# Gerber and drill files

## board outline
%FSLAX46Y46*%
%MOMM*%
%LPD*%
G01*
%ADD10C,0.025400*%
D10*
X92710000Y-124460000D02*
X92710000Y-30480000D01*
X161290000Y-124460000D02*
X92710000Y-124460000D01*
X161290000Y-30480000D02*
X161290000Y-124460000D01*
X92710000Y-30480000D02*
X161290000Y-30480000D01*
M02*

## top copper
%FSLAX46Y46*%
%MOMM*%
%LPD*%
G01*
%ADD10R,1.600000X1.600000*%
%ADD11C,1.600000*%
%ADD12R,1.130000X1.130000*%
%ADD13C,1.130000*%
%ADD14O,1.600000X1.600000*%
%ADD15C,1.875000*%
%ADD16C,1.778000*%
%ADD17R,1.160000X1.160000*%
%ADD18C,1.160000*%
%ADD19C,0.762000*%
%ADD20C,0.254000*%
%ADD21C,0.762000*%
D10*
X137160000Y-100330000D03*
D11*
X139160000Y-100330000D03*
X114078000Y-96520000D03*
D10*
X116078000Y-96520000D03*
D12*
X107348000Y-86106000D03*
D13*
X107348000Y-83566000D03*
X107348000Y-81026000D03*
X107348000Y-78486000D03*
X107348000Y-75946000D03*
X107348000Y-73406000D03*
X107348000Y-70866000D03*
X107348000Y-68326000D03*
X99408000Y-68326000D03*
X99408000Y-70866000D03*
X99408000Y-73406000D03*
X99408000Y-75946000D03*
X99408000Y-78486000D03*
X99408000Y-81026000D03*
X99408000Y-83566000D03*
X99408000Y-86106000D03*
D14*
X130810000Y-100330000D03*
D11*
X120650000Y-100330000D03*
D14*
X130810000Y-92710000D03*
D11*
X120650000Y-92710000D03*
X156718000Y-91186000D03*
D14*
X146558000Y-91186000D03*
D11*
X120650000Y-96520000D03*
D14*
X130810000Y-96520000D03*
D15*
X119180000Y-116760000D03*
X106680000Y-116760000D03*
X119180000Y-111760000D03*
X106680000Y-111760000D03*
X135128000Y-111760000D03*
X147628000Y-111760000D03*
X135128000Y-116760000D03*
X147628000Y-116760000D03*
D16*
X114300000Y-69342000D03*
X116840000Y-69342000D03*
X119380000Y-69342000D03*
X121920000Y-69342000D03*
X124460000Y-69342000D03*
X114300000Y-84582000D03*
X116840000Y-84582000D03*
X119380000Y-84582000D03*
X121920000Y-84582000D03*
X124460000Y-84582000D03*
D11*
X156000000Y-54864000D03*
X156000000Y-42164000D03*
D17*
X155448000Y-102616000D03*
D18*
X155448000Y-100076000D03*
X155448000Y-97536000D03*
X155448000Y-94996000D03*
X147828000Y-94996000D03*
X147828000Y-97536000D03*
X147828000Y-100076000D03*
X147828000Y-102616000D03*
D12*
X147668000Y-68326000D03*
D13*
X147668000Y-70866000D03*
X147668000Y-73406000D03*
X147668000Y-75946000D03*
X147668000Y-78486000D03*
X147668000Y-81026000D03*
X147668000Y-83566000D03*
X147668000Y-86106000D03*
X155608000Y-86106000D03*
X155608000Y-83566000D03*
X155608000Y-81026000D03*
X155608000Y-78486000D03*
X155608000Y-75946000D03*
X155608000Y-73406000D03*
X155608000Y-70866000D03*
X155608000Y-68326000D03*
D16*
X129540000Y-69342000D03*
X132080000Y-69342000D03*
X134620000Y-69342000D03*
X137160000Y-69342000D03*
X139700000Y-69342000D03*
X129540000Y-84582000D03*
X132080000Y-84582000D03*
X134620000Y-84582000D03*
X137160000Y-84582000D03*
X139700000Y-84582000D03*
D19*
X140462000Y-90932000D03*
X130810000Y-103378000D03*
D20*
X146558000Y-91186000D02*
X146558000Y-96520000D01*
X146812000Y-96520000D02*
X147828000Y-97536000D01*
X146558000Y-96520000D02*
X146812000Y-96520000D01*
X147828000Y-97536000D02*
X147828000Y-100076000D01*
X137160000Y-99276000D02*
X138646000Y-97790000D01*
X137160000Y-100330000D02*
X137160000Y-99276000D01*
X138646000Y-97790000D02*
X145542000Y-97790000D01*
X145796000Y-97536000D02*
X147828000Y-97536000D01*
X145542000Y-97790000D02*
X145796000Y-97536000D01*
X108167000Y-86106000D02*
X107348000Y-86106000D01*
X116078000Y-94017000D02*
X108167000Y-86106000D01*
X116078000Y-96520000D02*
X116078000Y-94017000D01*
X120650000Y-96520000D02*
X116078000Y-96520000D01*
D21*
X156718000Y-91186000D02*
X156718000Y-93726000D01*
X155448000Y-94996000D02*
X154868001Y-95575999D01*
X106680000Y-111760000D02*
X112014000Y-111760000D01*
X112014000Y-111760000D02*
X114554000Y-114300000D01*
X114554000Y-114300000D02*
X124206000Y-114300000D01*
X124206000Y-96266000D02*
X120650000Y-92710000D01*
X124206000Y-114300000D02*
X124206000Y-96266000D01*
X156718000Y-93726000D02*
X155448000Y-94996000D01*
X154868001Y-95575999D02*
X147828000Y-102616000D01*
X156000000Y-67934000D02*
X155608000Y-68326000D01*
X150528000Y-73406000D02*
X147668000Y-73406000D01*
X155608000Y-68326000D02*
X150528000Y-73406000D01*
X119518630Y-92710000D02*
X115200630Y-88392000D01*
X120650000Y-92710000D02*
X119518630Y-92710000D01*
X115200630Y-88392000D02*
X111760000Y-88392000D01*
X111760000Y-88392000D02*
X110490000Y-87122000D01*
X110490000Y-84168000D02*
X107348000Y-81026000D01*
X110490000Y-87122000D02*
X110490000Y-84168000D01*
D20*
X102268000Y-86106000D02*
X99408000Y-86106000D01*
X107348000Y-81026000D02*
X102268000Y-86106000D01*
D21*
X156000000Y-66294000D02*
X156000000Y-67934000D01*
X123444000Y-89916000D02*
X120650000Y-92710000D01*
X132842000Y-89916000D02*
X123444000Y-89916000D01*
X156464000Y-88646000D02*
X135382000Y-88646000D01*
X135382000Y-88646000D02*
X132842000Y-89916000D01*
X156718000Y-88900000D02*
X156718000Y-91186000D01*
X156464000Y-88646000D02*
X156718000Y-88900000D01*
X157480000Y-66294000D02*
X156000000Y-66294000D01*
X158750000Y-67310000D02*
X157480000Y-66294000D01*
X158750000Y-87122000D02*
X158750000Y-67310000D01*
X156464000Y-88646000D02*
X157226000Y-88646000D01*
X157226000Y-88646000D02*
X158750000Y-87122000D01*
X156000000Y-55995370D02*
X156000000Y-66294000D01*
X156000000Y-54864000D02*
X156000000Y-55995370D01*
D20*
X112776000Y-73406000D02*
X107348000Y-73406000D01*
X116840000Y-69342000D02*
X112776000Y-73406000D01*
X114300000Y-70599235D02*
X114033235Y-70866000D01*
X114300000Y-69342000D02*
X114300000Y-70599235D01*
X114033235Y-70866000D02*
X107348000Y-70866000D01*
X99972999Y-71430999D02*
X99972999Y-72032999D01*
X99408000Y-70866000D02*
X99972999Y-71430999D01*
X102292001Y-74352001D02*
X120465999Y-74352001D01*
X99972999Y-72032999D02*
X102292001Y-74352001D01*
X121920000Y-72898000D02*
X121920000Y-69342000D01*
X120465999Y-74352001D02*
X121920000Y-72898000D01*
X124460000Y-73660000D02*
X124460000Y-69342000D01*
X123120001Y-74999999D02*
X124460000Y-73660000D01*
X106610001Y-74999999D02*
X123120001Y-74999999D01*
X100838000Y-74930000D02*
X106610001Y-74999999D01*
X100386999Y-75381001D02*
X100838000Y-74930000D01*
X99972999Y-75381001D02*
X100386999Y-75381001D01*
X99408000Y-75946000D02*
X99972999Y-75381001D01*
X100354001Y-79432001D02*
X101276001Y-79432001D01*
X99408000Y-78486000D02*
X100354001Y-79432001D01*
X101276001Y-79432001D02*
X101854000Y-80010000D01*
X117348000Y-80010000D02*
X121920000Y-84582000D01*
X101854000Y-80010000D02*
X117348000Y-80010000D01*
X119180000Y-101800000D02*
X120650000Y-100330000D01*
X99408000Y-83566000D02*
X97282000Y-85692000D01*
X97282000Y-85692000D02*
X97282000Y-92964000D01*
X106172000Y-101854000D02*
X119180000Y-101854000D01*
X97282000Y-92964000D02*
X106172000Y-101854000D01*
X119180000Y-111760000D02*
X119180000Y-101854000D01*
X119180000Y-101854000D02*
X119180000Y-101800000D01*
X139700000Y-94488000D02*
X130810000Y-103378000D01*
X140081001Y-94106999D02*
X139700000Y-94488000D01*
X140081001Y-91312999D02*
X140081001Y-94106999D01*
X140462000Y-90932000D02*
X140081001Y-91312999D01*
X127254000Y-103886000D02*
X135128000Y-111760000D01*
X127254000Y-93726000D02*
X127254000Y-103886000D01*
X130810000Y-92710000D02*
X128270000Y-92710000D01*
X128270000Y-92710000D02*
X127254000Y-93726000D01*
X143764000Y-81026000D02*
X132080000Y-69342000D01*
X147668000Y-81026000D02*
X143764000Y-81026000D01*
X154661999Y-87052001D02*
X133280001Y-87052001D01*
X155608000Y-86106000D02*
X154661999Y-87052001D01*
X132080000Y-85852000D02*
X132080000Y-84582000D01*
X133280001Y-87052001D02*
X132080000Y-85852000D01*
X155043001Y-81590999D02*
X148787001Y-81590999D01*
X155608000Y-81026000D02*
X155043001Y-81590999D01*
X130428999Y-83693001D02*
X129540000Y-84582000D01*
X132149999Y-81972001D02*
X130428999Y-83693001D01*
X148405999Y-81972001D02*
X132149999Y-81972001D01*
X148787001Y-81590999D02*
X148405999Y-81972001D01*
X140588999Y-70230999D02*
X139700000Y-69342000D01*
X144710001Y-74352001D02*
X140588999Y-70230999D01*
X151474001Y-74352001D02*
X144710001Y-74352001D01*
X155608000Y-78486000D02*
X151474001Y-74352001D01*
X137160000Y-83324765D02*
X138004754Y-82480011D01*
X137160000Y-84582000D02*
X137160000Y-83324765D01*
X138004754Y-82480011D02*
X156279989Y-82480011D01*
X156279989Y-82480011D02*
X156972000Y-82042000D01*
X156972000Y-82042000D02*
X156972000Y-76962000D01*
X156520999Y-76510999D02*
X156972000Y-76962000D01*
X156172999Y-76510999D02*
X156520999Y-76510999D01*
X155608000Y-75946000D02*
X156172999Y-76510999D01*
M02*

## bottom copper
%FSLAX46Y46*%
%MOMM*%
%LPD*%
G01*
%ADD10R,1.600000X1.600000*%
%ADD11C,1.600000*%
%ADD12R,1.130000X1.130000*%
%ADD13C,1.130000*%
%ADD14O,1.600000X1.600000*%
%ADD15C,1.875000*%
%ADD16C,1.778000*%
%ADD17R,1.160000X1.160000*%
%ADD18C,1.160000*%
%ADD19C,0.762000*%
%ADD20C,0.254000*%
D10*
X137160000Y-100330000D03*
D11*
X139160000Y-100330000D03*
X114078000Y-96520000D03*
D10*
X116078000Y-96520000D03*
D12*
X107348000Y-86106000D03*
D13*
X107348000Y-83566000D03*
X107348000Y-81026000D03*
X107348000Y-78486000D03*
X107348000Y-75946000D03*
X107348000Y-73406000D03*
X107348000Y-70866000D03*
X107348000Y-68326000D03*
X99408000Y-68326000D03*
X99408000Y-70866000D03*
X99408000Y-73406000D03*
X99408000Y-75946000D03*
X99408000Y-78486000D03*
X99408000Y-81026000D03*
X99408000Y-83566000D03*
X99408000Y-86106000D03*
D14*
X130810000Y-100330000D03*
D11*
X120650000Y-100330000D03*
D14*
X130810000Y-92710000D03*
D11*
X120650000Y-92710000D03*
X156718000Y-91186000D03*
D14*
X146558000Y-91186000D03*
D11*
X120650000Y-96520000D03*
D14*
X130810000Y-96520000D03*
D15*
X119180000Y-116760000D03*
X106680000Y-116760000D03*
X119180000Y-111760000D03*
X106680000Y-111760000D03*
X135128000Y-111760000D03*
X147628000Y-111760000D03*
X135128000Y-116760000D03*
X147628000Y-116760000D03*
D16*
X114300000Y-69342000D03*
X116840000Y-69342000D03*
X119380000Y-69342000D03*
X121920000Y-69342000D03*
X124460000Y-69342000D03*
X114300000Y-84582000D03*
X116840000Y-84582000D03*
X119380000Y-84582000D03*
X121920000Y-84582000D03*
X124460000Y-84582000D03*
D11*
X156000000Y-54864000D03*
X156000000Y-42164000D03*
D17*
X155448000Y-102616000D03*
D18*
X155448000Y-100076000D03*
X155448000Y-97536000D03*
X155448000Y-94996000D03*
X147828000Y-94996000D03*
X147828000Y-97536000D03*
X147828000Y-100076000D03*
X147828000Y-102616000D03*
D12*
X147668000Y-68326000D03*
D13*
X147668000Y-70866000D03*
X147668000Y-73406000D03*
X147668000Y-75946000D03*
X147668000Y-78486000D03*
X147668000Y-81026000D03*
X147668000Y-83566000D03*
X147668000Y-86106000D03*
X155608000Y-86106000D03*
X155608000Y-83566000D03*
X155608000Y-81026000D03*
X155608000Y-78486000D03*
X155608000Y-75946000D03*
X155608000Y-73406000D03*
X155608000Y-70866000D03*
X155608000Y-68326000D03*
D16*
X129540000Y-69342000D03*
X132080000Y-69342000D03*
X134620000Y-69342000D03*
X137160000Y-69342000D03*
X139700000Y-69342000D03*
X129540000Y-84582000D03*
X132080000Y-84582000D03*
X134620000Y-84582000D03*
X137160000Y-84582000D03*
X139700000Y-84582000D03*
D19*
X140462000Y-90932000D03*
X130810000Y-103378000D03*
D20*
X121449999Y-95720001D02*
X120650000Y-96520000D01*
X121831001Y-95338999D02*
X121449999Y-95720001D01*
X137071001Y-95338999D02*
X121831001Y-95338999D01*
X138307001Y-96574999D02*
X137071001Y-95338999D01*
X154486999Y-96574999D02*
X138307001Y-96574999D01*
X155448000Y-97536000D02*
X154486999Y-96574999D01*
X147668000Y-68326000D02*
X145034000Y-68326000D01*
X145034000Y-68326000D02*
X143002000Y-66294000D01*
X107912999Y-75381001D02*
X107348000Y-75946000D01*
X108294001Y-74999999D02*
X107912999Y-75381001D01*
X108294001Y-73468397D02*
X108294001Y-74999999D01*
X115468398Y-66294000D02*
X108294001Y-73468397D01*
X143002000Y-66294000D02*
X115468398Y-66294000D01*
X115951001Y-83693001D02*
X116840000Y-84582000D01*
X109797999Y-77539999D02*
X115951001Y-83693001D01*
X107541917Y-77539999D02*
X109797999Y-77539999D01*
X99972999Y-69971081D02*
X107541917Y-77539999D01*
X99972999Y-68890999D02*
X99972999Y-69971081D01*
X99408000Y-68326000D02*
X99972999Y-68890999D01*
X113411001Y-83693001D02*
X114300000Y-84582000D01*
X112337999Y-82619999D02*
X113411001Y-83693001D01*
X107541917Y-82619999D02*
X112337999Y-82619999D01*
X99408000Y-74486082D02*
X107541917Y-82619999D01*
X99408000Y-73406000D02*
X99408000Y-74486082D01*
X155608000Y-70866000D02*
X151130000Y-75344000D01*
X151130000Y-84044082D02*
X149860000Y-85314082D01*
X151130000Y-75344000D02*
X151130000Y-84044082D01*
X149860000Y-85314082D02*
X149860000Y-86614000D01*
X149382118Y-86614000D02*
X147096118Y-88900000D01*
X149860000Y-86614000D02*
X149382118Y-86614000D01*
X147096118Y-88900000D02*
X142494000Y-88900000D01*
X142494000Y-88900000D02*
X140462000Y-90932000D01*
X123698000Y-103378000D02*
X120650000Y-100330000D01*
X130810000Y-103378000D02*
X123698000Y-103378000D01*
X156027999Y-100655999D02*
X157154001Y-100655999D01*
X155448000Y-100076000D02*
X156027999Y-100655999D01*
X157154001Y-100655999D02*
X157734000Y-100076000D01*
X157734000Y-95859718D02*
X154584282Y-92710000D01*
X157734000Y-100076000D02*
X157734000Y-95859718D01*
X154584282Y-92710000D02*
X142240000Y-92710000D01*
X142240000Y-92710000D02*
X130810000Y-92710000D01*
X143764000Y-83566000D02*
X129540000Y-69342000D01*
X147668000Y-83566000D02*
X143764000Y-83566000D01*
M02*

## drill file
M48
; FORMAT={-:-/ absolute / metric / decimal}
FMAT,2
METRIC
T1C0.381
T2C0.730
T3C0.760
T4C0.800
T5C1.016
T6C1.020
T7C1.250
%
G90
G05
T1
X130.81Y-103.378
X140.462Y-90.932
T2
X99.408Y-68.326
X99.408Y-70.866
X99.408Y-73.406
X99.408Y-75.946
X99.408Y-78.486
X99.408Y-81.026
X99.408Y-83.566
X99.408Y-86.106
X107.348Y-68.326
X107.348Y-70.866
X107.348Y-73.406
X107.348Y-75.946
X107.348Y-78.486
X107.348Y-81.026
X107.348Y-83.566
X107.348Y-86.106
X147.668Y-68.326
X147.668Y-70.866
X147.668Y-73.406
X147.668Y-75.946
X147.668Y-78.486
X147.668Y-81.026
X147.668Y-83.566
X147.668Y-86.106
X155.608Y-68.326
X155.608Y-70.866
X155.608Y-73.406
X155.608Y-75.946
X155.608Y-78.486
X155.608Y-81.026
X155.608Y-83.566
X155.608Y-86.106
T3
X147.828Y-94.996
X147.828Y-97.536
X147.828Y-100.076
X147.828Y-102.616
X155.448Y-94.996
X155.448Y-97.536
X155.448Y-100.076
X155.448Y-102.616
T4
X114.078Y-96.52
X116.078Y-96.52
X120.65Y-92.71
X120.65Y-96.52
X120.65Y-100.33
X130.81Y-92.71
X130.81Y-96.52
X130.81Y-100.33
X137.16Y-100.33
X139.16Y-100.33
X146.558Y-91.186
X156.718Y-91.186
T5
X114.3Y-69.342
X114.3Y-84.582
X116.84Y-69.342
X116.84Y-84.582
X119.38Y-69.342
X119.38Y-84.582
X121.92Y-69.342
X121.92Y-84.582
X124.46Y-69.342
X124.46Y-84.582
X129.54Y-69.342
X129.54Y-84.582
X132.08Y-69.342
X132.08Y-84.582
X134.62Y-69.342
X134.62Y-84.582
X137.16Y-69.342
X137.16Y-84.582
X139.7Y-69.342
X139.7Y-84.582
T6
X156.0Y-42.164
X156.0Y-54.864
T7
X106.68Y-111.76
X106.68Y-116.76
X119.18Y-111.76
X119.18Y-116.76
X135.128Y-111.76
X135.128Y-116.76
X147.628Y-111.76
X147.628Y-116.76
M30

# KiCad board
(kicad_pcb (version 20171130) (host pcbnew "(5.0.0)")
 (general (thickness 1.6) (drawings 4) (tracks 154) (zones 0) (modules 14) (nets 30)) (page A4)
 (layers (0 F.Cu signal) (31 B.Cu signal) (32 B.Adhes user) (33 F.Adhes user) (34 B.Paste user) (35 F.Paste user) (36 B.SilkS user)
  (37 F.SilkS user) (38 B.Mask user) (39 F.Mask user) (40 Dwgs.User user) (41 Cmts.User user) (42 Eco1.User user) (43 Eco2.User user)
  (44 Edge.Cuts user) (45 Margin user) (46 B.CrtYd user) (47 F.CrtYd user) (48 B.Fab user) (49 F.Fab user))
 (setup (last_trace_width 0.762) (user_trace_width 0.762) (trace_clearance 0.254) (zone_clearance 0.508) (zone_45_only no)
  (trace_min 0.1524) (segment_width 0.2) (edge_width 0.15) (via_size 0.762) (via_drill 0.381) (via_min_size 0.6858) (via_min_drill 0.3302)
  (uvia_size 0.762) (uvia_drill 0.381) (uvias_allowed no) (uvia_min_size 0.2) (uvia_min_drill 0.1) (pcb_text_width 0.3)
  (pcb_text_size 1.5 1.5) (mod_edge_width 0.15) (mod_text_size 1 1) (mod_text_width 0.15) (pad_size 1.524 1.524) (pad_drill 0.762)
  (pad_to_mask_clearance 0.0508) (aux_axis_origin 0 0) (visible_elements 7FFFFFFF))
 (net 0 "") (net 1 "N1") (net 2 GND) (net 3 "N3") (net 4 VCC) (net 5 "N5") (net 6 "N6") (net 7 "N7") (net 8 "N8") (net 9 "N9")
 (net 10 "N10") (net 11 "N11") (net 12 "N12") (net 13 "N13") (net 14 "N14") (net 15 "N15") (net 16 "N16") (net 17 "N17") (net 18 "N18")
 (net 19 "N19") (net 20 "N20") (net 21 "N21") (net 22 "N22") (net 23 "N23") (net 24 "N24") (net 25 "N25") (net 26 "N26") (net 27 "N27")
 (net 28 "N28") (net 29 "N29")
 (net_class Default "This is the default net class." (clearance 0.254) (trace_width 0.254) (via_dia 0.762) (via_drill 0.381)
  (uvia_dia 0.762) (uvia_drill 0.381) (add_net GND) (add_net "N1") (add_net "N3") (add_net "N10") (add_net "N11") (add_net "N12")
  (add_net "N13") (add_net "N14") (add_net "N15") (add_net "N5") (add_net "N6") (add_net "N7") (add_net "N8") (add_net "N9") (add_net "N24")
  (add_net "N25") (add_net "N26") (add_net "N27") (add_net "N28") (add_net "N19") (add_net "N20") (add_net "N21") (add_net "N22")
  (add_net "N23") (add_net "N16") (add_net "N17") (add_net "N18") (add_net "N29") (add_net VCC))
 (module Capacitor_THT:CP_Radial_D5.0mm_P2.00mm (layer F.Cu) (at 137.16 100.33)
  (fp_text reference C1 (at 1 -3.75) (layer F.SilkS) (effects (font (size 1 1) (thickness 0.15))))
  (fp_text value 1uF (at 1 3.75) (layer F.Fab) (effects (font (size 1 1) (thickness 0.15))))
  (pad 1 thru_hole rect (at 0 0) (size 1.6 1.6) (drill 0.8) (layers *.Cu *.Mask) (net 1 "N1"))
  (pad 2 thru_hole circle (at 2 0) (size 1.6 1.6) (drill 0.8) (layers *.Cu *.Mask) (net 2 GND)))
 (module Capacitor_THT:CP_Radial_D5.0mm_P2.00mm (layer F.Cu) (at 116.078 96.52 180)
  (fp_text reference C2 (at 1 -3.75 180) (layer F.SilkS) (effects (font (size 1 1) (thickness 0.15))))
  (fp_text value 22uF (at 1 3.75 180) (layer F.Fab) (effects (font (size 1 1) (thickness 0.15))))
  (pad 2 thru_hole circle (at 2 0 180) (size 1.6 1.6) (drill 0.8) (layers *.Cu *.Mask) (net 2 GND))
  (pad 1 thru_hole rect (at 0 0 180) (size 1.6 1.6) (drill 0.8) (layers *.Cu *.Mask) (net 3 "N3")))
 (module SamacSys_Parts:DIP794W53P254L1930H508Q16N (layer F.Cu) (at 103.378 77.216 180)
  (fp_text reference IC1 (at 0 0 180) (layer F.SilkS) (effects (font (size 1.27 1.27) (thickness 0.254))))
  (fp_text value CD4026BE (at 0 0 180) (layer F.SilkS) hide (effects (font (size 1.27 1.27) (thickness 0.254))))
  (pad 1 thru_hole rect (at -3.97 -8.89 180) (size 1.13 1.13) (drill 0.73) (layers *.Cu *.Mask) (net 3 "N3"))
  (pad 2 thru_hole circle (at -3.97 -6.35 180) (size 1.13 1.13) (drill 0.73) (layers *.Cu *.Mask) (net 2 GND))
  (pad 3 thru_hole circle (at -3.97 -3.81 180) (size 1.13 1.13) (drill 0.73) (layers *.Cu *.Mask) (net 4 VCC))
  (pad 4 thru_hole circle (at -3.97 -1.27 180) (size 1.13 1.13) (drill 0.73) (layers *.Cu *.Mask) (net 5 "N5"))
  (pad 5 thru_hole circle (at -3.97 1.27 180) (size 1.13 1.13) (drill 0.73) (layers *.Cu *.Mask) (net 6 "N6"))
  (pad 6 thru_hole circle (at -3.97 3.81 180) (size 1.13 1.13) (drill 0.73) (layers *.Cu *.Mask) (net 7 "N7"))
  (pad 7 thru_hole circle (at -3.97 6.35 180) (size 1.13 1.13) (drill 0.73) (layers *.Cu *.Mask) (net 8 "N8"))
  (pad 8 thru_hole circle (at -3.97 8.89 180) (size 1.13 1.13) (drill 0.73) (layers *.Cu *.Mask) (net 2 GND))
  (pad 9 thru_hole circle (at 3.97 8.89 180) (size 1.13 1.13) (drill 0.73) (layers *.Cu *.Mask) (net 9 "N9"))
  (pad 10 thru_hole circle (at 3.97 6.35 180) (size 1.13 1.13) (drill 0.73) (layers *.Cu *.Mask) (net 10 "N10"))
  (pad 11 thru_hole circle (at 3.97 3.81 180) (size 1.13 1.13) (drill 0.73) (layers *.Cu *.Mask) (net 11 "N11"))
  (pad 12 thru_hole circle (at 3.97 1.27 180) (size 1.13 1.13) (drill 0.73) (layers *.Cu *.Mask) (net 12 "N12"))
  (pad 13 thru_hole circle (at 3.97 -1.27 180) (size 1.13 1.13) (drill 0.73) (layers *.Cu *.Mask) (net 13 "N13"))
  (pad 14 thru_hole circle (at 3.97 -3.81 180) (size 1.13 1.13) (drill 0.73) (layers *.Cu *.Mask) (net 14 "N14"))
  (pad 15 thru_hole circle (at 3.97 -6.35 180) (size 1.13 1.13) (drill 0.73) (layers *.Cu *.Mask) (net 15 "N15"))
  (pad 16 thru_hole circle (at 3.97 -8.89 180) (size 1.13 1.13) (drill 0.73) (layers *.Cu *.Mask) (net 4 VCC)))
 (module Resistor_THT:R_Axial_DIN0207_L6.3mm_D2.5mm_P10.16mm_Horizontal (layer F.Cu) (at 120.65 100.33)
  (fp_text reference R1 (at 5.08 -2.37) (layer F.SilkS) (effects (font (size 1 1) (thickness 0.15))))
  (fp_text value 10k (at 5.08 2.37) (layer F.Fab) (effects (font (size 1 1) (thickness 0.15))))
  (pad 2 thru_hole oval (at 10.16 0) (size 1.6 1.6) (drill 0.8) (layers *.Cu *.Mask) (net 2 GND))
  (pad 1 thru_hole circle (at 0 0) (size 1.6 1.6) (drill 0.8) (layers *.Cu *.Mask) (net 15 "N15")))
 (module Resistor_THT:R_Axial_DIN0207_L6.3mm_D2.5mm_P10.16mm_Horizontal (layer F.Cu) (at 120.65 92.71)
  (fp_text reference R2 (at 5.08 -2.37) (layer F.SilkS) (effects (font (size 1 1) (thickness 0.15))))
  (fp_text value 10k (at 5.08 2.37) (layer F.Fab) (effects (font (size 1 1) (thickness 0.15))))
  (pad 2 thru_hole oval (at 10.16 0) (size 1.6 1.6) (drill 0.8) (layers *.Cu *.Mask) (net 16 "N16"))
  (pad 1 thru_hole circle (at 0 0) (size 1.6 1.6) (drill 0.8) (layers *.Cu *.Mask) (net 4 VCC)))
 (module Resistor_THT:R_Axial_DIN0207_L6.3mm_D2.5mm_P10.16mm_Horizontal (layer F.Cu) (at 156.718 91.186 180)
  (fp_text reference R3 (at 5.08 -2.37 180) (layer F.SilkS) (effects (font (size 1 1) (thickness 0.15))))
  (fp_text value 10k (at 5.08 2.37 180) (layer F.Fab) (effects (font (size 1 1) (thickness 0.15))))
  (pad 1 thru_hole circle (at 0 0 180) (size 1.6 1.6) (drill 0.8) (layers *.Cu *.Mask) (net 4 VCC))
  (pad 2 thru_hole oval (at 10.16 0 180) (size 1.6 1.6) (drill 0.8) (layers *.Cu *.Mask) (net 1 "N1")))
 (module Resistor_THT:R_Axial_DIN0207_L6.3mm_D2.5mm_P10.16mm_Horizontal (layer F.Cu) (at 120.65 96.52)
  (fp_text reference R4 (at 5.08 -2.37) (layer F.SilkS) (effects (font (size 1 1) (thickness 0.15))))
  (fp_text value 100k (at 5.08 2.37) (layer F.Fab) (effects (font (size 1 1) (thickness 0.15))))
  (pad 1 thru_hole circle (at 0 0) (size 1.6 1.6) (drill 0.8) (layers *.Cu *.Mask) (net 3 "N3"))
  (pad 2 thru_hole oval (at 10.16 0) (size 1.6 1.6) (drill 0.8) (layers *.Cu *.Mask) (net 2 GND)))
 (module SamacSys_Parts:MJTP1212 (layer F.Cu) (at 106.68 111.76)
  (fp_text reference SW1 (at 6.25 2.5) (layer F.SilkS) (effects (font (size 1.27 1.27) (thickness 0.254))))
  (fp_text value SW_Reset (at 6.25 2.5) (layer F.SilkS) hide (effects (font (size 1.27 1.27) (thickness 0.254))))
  (pad 4 thru_hole circle (at 12.5 5) (size 1.875 1.875) (drill 1.25) (layers *.Cu *.Mask))
  (pad 3 thru_hole circle (at 0 5) (size 1.875 1.875) (drill 1.25) (layers *.Cu *.Mask))
  (pad 2 thru_hole circle (at 12.5 0) (size 1.875 1.875) (drill 1.25) (layers *.Cu *.Mask) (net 15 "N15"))
  (pad 1 thru_hole circle (at 0 0) (size 1.875 1.875) (drill 1.25) (layers *.Cu *.Mask) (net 4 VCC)))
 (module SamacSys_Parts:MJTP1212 (layer F.Cu) (at 135.128 111.76)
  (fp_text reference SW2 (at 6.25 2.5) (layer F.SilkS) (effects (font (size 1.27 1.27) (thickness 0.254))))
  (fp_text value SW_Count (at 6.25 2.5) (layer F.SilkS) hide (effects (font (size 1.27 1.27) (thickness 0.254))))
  (pad 1 thru_hole circle (at 0 0) (size 1.875 1.875) (drill 1.25) (layers *.Cu *.Mask) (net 16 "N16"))
  (pad 2 thru_hole circle (at 12.5 0) (size 1.875 1.875) (drill 1.25) (layers *.Cu *.Mask) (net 2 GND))
  (pad 3 thru_hole circle (at 0 5) (size 1.875 1.875) (drill 1.25) (layers *.Cu *.Mask))
  (pad 4 thru_hole circle (at 12.5 5) (size 1.875 1.875) (drill 1.25) (layers *.Cu *.Mask)))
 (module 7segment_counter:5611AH (layer F.Cu) (at 119.38 76.962)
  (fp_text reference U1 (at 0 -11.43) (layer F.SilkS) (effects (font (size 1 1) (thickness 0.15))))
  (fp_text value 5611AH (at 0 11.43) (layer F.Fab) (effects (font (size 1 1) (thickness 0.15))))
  (pad 1 thru_hole circle (at -5.08 -7.62) (size 1.778 1.778) (drill 1.016) (layers *.Cu *.Mask) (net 8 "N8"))
  (pad 2 thru_hole circle (at -2.54 -7.62) (size 1.778 1.778) (drill 1.016) (layers *.Cu *.Mask) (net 7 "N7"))
  (pad 3 thru_hole circle (at 0 -7.62) (size 1.778 1.778) (drill 1.016) (layers *.Cu *.Mask) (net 2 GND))
  (pad 4 thru_hole circle (at 2.54 -7.62) (size 1.778 1.778) (drill 1.016) (layers *.Cu *.Mask) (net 10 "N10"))
  (pad 5 thru_hole circle (at 5.08 -7.62) (size 1.778 1.778) (drill 1.016) (layers *.Cu *.Mask) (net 12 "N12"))
  (pad 6 thru_hole circle (at -5.08 7.62) (size 1.778 1.778) (drill 1.016) (layers *.Cu *.Mask) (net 11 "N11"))
  (pad 7 thru_hole circle (at -2.54 7.62) (size 1.778 1.778) (drill 1.016) (layers *.Cu *.Mask) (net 9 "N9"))
  (pad 8 thru_hole circle (at 0 7.62) (size 1.778 1.778) (drill 1.016) (layers *.Cu *.Mask) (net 2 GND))
  (pad 9 thru_hole circle (at 2.54 7.62) (size 1.778 1.778) (drill 1.016) (layers *.Cu *.Mask) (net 13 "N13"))
  (pad 10 thru_hole circle (at 5.08 7.62) (size 1.778 1.778) (drill 1.016) (layers *.Cu *.Mask) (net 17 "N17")))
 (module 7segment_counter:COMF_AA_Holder (layer F.Cu) (at 127 48.514)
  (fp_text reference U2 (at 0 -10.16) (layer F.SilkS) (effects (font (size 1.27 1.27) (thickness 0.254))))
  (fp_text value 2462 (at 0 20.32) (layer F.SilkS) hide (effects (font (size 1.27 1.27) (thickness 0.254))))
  (pad 1 thru_hole circle (at 29 6.35) (size 1.6 1.6) (drill 1.02) (layers *.Cu *.Mask) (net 4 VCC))
  (pad 2 thru_hole circle (at 29 -6.35) (size 1.6 1.6) (drill 1.02) (layers *.Cu *.Mask) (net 2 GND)))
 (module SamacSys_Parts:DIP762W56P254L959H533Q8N (layer F.Cu) (at 151.638 98.806 180)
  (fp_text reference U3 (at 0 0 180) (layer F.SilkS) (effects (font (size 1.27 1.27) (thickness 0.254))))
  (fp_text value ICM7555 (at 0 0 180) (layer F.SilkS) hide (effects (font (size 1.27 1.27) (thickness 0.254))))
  (pad 1 thru_hole rect (at -3.81 -3.81 180) (size 1.16 1.16) (drill 0.76) (layers *.Cu *.Mask) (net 2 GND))
  (pad 2 thru_hole circle (at -3.81 -1.27 180) (size 1.16 1.16) (drill 0.76) (layers *.Cu *.Mask) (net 16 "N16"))
  (pad 3 thru_hole circle (at -3.81 1.27 180) (size 1.16 1.16) (drill 0.76) (layers *.Cu *.Mask) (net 3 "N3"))
  (pad 4 thru_hole circle (at -3.81 3.81 180) (size 1.16 1.16) (drill 0.76) (layers *.Cu *.Mask) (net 4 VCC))
  (pad 5 thru_hole circle (at 3.81 3.81 180) (size 1.16 1.16) (drill 0.76) (layers *.Cu *.Mask) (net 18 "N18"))
  (pad 6 thru_hole circle (at 3.81 1.27 180) (size 1.16 1.16) (drill 0.76) (layers *.Cu *.Mask) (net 1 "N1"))
  (pad 7 thru_hole circle (at 3.81 -1.27 180) (size 1.16 1.16) (drill 0.76) (layers *.Cu *.Mask) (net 1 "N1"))
  (pad 8 thru_hole circle (at 3.81 -3.81 180) (size 1.16 1.16) (drill 0.76) (layers *.Cu *.Mask) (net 4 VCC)))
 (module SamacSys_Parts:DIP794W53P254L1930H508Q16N (layer F.Cu) (at 151.638 77.216)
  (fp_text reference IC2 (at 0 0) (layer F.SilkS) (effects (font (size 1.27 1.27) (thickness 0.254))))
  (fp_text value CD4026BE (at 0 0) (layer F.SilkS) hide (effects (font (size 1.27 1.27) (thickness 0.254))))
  (pad 1 thru_hole rect (at -3.97 -8.89) (size 1.13 1.13) (drill 0.73) (layers *.Cu *.Mask) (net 6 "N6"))
  (pad 2 thru_hole circle (at -3.97 -6.35) (size 1.13 1.13) (drill 0.73) (layers *.Cu *.Mask) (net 2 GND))
  (pad 3 thru_hole circle (at -3.97 -3.81) (size 1.13 1.13) (drill 0.73) (layers *.Cu *.Mask) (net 4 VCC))
  (pad 4 thru_hole circle (at -3.97 -1.27) (size 1.13 1.13) (drill 0.73) (layers *.Cu *.Mask) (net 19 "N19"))
  (pad 5 thru_hole circle (at -3.97 1.27) (size 1.13 1.13) (drill 0.73) (layers *.Cu *.Mask) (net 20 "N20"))
  (pad 6 thru_hole circle (at -3.97 3.81) (size 1.13 1.13) (drill 0.73) (layers *.Cu *.Mask) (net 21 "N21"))
  (pad 7 thru_hole circle (at -3.97 6.35) (size 1.13 1.13) (drill 0.73) (layers *.Cu *.Mask) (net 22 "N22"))
  (pad 8 thru_hole circle (at -3.97 8.89) (size 1.13 1.13) (drill 0.73) (layers *.Cu *.Mask) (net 2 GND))
  (pad 9 thru_hole circle (at 3.97 8.89) (size 1.13 1.13) (drill 0.73) (layers *.Cu *.Mask) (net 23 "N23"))
  (pad 10 thru_hole circle (at 3.97 6.35) (size 1.13 1.13) (drill 0.73) (layers *.Cu *.Mask) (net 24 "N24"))
  (pad 11 thru_hole circle (at 3.97 3.81) (size 1.13 1.13) (drill 0.73) (layers *.Cu *.Mask) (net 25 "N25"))
  (pad 12 thru_hole circle (at 3.97 1.27) (size 1.13 1.13) (drill 0.73) (layers *.Cu *.Mask) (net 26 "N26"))
  (pad 13 thru_hole circle (at 3.97 -1.27) (size 1.13 1.13) (drill 0.73) (layers *.Cu *.Mask) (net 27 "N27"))
  (pad 14 thru_hole circle (at 3.97 -3.81) (size 1.13 1.13) (drill 0.73) (layers *.Cu *.Mask) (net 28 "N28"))
  (pad 15 thru_hole circle (at 3.97 -6.35) (size 1.13 1.13) (drill 0.73) (layers *.Cu *.Mask) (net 15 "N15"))
  (pad 16 thru_hole circle (at 3.97 -8.89) (size 1.13 1.13) (drill 0.73) (layers *.Cu *.Mask) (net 4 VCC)))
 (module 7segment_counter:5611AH (layer F.Cu) (at 134.62 76.962)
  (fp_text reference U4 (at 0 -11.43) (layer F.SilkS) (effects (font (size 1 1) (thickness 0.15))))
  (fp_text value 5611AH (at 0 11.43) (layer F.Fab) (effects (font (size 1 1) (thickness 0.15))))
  (pad 1 thru_hole circle (at -5.08 -7.62) (size 1.778 1.778) (drill 1.016) (layers *.Cu *.Mask) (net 22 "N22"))
  (pad 2 thru_hole circle (at -2.54 -7.62) (size 1.778 1.778) (drill 1.016) (layers *.Cu *.Mask) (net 21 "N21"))
  (pad 3 thru_hole circle (at 0 -7.62) (size 1.778 1.778) (drill 1.016) (layers *.Cu *.Mask) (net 2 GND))
  (pad 4 thru_hole circle (at 2.54 -7.62) (size 1.778 1.778) (drill 1.016) (layers *.Cu *.Mask) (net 24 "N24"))
  (pad 5 thru_hole circle (at 5.08 -7.62) (size 1.778 1.778) (drill 1.016) (layers *.Cu *.Mask) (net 26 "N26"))
  (pad 6 thru_hole circle (at -5.08 7.62) (size 1.778 1.778) (drill 1.016) (layers *.Cu *.Mask) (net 25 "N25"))
  (pad 7 thru_hole circle (at -2.54 7.62) (size 1.778 1.778) (drill 1.016) (layers *.Cu *.Mask) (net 23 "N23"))
  (pad 8 thru_hole circle (at 0 7.62) (size 1.778 1.778) (drill 1.016) (layers *.Cu *.Mask) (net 2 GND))
  (pad 9 thru_hole circle (at 2.54 7.62) (size 1.778 1.778) (drill 1.016) (layers *.Cu *.Mask) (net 27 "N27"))
  (pad 10 thru_hole circle (at 5.08 7.62) (size 1.778 1.778) (drill 1.016) (layers *.Cu *.Mask) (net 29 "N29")))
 (gr_line (start 92.71 124.46) (end 92.71 30.48) (layer Edge.Cuts) (width 0.0254))
 (gr_line (start 161.29 124.46) (end 92.71 124.46) (layer Edge.Cuts) (width 0.0254))
 (gr_line (start 161.29 30.48) (end 161.29 124.46) (layer Edge.Cuts) (width 0.0254))
 (gr_line (start 92.71 30.48) (end 161.29 30.48) (layer Edge.Cuts) (width 0.0254))
 (segment (start 146.558 91.186) (end 146.558 96.52) (width 0.254) (layer F.Cu) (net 1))
 (segment (start 146.812 96.52) (end 147.828 97.536) (width 0.254) (layer F.Cu) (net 1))
 (segment (start 146.558 96.52) (end 146.812 96.52) (width 0.254) (layer F.Cu) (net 1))
 (segment (start 147.828 97.536) (end 147.828 100.076) (width 0.254) (layer F.Cu) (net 1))
 (segment (start 137.16 99.276) (end 138.646 97.79) (width 0.254) (layer F.Cu) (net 1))
 (segment (start 137.16 100.33) (end 137.16 99.276) (width 0.254) (layer F.Cu) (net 1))
 (segment (start 138.646 97.79) (end 145.542 97.79) (width 0.254) (layer F.Cu) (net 1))
 (segment (start 145.796 97.536) (end 147.828 97.536) (width 0.254) (layer F.Cu) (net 1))
 (segment (start 145.542 97.79) (end 145.796 97.536) (width 0.254) (layer F.Cu) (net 1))
 (segment (start 121.449999 95.720001) (end 120.65 96.52) (width 0.254) (layer B.Cu) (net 3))
 (segment (start 121.831001 95.338999) (end 121.449999 95.720001) (width 0.254) (layer B.Cu) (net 3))
 (segment (start 137.071001 95.338999) (end 121.831001 95.338999) (width 0.254) (layer B.Cu) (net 3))
 (segment (start 108.167 86.106) (end 107.348 86.106) (width 0.254) (layer F.Cu) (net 3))
 (segment (start 116.078 94.017) (end 108.167 86.106) (width 0.254) (layer F.Cu) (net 3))
 (segment (start 116.078 96.52) (end 116.078 94.017) (width 0.254) (layer F.Cu) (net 3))
 (segment (start 120.65 96.52) (end 116.078 96.52) (width 0.254) (layer F.Cu) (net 3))
 (segment (start 138.307001 96.574999) (end 137.071001 95.338999) (width 0.254) (layer B.Cu) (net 3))
 (segment (start 154.486999 96.574999) (end 138.307001 96.574999) (width 0.254) (layer B.Cu) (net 3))
 (segment (start 155.448 97.536) (end 154.486999 96.574999) (width 0.254) (layer B.Cu) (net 3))
 (segment (start 156.718 91.186) (end 156.718 93.726) (width 0.762) (layer F.Cu) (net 4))
 (segment (start 155.448 94.996) (end 154.868001 95.575999) (width 0.762) (layer F.Cu) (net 4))
 (segment (start 106.68 111.76) (end 112.014 111.76) (width 0.762) (layer F.Cu) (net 4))
 (segment (start 112.014 111.76) (end 114.554 114.3) (width 0.762) (layer F.Cu) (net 4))
 (segment (start 114.554 114.3) (end 124.206 114.3) (width 0.762) (layer F.Cu) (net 4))
 (segment (start 124.206 96.266) (end 120.65 92.71) (width 0.762) (layer F.Cu) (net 4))
 (segment (start 124.206 114.3) (end 124.206 96.266) (width 0.762) (layer F.Cu) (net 4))
 (segment (start 156.718 93.726) (end 155.448 94.996) (width 0.762) (layer F.Cu) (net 4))
 (segment (start 154.868001 95.575999) (end 147.828 102.616) (width 0.762) (layer F.Cu) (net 4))
 (segment (start 156 67.934) (end 155.608 68.326) (width 0.762) (layer F.Cu) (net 4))
 (segment (start 150.528 73.406) (end 147.668 73.406) (width 0.762) (layer F.Cu) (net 4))
 (segment (start 155.608 68.326) (end 150.528 73.406) (width 0.762) (layer F.Cu) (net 4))
 (segment (start 119.51863 92.71) (end 115.20063 88.392) (width 0.762) (layer F.Cu) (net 4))
 (segment (start 120.65 92.71) (end 119.51863 92.71) (width 0.762) (layer F.Cu) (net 4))
 (segment (start 115.20063 88.392) (end 111.76 88.392) (width 0.762) (layer F.Cu) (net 4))
 (segment (start 111.76 88.392) (end 110.49 87.122) (width 0.762) (layer F.Cu) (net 4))
 (segment (start 110.49 84.168) (end 107.348 81.026) (width 0.762) (layer F.Cu) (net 4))
 (segment (start 110.49 87.122) (end 110.49 84.168) (width 0.762) (layer F.Cu) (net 4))
 (segment (start 102.268 86.106) (end 99.408 86.106) (width 0.254) (layer F.Cu) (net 4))
 (segment (start 107.348 81.026) (end 102.268 86.106) (width 0.254) (layer F.Cu) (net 4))
 (segment (start 156 66.294) (end 156 67.934) (width 0.762) (layer F.Cu) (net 4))
 (segment (start 123.444 89.916) (end 120.65 92.71) (width 0.762) (layer F.Cu) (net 4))
 (segment (start 132.842 89.916) (end 123.444 89.916) (width 0.762) (layer F.Cu) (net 4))
 (segment (start 156.464 88.646) (end 135.382 88.646) (width 0.762) (layer F.Cu) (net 4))
 (segment (start 135.382 88.646) (end 132.842 89.916) (width 0.762) (layer F.Cu) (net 4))
 (segment (start 156.718 88.9) (end 156.718 91.186) (width 0.762) (layer F.Cu) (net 4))
 (segment (start 156.464 88.646) (end 156.718 88.9) (width 0.762) (layer F.Cu) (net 4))
 (segment (start 157.48 66.294) (end 156 66.294) (width 0.762) (layer F.Cu) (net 4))
 (segment (start 158.75 67.31) (end 157.48 66.294) (width 0.762) (layer F.Cu) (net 4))
 (segment (start 158.75 87.122) (end 158.75 67.31) (width 0.762) (layer F.Cu) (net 4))
 (segment (start 156.464 88.646) (end 157.226 88.646) (width 0.762) (layer F.Cu) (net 4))
 (segment (start 157.226 88.646) (end 158.75 87.122) (width 0.762) (layer F.Cu) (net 4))
 (segment (start 156 55.99537) (end 156 66.294) (width 0.762) (layer F.Cu) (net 4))
 (segment (start 156 54.864) (end 156 55.99537) (width 0.762) (layer F.Cu) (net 4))
 (segment (start 147.668 68.326) (end 145.034 68.326) (width 0.254) (layer B.Cu) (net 6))
 (segment (start 145.034 68.326) (end 143.002 66.294) (width 0.254) (layer B.Cu) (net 6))
 (segment (start 107.912999 75.381001) (end 107.348 75.946) (width 0.254) (layer B.Cu) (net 6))
 (segment (start 108.294001 74.999999) (end 107.912999 75.381001) (width 0.254) (layer B.Cu) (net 6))
 (segment (start 108.294001 73.468397) (end 108.294001 74.999999) (width 0.254) (layer B.Cu) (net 6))
 (segment (start 115.468398 66.294) (end 108.294001 73.468397) (width 0.254) (layer B.Cu) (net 6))
 (segment (start 143.002 66.294) (end 115.468398 66.294) (width 0.254) (layer B.Cu) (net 6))
 (segment (start 112.776 73.406) (end 107.348 73.406) (width 0.254) (layer F.Cu) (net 7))
 (segment (start 116.84 69.342) (end 112.776 73.406) (width 0.254) (layer F.Cu) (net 7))
 (segment (start 114.3 70.599235) (end 114.033235 70.866) (width 0.254) (layer F.Cu) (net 8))
 (segment (start 114.3 69.342) (end 114.3 70.599235) (width 0.254) (layer F.Cu) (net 8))
 (segment (start 114.033235 70.866) (end 107.348 70.866) (width 0.254) (layer F.Cu) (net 8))
 (segment (start 115.951001 83.693001) (end 116.84 84.582) (width 0.254) (layer B.Cu) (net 9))
 (segment (start 109.797999 77.539999) (end 115.951001 83.693001) (width 0.254) (layer B.Cu) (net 9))
 (segment (start 107.541917 77.539999) (end 109.797999 77.539999) (width 0.254) (layer B.Cu) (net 9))
 (segment (start 99.972999 69.971081) (end 107.541917 77.539999) (width 0.254) (layer B.Cu) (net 9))
 (segment (start 99.972999 68.890999) (end 99.972999 69.971081) (width 0.254) (layer B.Cu) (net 9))
 (segment (start 99.408 68.326) (end 99.972999 68.890999) (width 0.254) (layer B.Cu) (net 9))
 (segment (start 99.972999 71.430999) (end 99.972999 72.032999) (width 0.254) (layer F.Cu) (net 10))
 (segment (start 99.408 70.866) (end 99.972999 71.430999) (width 0.254) (layer F.Cu) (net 10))
 (segment (start 102.292001 74.352001) (end 120.465999 74.352001) (width 0.254) (layer F.Cu) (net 10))
 (segment (start 99.972999 72.032999) (end 102.292001 74.352001) (width 0.254) (layer F.Cu) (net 10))
 (segment (start 121.92 72.898) (end 121.92 69.342) (width 0.254) (layer F.Cu) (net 10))
 (segment (start 120.465999 74.352001) (end 121.92 72.898) (width 0.254) (layer F.Cu) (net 10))
 (segment (start 113.411001 83.693001) (end 114.3 84.582) (width 0.254) (layer B.Cu) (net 11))
 (segment (start 112.337999 82.619999) (end 113.411001 83.693001) (width 0.254) (layer B.Cu) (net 11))
 (segment (start 107.541917 82.619999) (end 112.337999 82.619999) (width 0.254) (layer B.Cu) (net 11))
 (segment (start 99.408 74.486082) (end 107.541917 82.619999) (width 0.254) (layer B.Cu) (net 11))
 (segment (start 99.408 73.406) (end 99.408 74.486082) (width 0.254) (layer B.Cu) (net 11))
 (segment (start 124.46 73.66) (end 124.46 69.342) (width 0.254) (layer F.Cu) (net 12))
 (segment (start 123.120001 74.999999) (end 124.46 73.66) (width 0.254) (layer F.Cu) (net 12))
 (segment (start 106.610001 74.999999) (end 123.120001 74.999999) (width 0.254) (layer F.Cu) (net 12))
 (segment (start 100.838 74.93) (end 106.610001 74.999999) (width 0.254) (layer F.Cu) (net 12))
 (segment (start 100.386999 75.381001) (end 100.838 74.93) (width 0.254) (layer F.Cu) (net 12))
 (segment (start 99.972999 75.381001) (end 100.386999 75.381001) (width 0.254) (layer F.Cu) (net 12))
 (segment (start 99.408 75.946) (end 99.972999 75.381001) (width 0.254) (layer F.Cu) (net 12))
 (segment (start 100.354001 79.432001) (end 101.276001 79.432001) (width 0.254) (layer F.Cu) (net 13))
 (segment (start 99.408 78.486) (end 100.354001 79.432001) (width 0.254) (layer F.Cu) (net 13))
 (segment (start 101.276001 79.432001) (end 101.854 80.01) (width 0.254) (layer F.Cu) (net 13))
 (segment (start 117.348 80.01) (end 121.92 84.582) (width 0.254) (layer F.Cu) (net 13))
 (segment (start 101.854 80.01) (end 117.348 80.01) (width 0.254) (layer F.Cu) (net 13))
 (segment (start 119.18 101.8) (end 120.65 100.33) (width 0.254) (layer F.Cu) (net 15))
 (segment (start 99.408 83.566) (end 97.282 85.692) (width 0.254) (layer F.Cu) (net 15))
 (segment (start 97.282 85.692) (end 97.282 92.964) (width 0.254) (layer F.Cu) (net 15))
 (segment (start 106.172 101.854) (end 119.18 101.854) (width 0.254) (layer F.Cu) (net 15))
 (segment (start 97.282 92.964) (end 106.172 101.854) (width 0.254) (layer F.Cu) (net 15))
 (segment (start 119.18 111.76) (end 119.18 101.854) (width 0.254) (layer F.Cu) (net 15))
 (segment (start 119.18 101.854) (end 119.18 101.8) (width 0.254) (layer F.Cu) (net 15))
 (segment (start 155.608 70.866) (end 151.13 75.344) (width 0.254) (layer B.Cu) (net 15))
 (segment (start 151.13 84.044082) (end 149.86 85.314082) (width 0.254) (layer B.Cu) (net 15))
 (segment (start 151.13 75.344) (end 151.13 84.044082) (width 0.254) (layer B.Cu) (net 15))
 (segment (start 149.86 85.314082) (end 149.86 86.614) (width 0.254) (layer B.Cu) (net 15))
 (segment (start 149.382118 86.614) (end 147.096118 88.9) (width 0.254) (layer B.Cu) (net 15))
 (segment (start 149.86 86.614) (end 149.382118 86.614) (width 0.254) (layer B.Cu) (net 15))
 (segment (start 147.096118 88.9) (end 142.494 88.9) (width 0.254) (layer B.Cu) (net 15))
 (segment (start 142.494 88.9) (end 140.462 90.932) (width 0.254) (layer B.Cu) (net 15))
 (via (at 140.462 90.932) (size 0.762) (drill 0.381) (layers F.Cu B.Cu) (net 15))
 (segment (start 139.7 94.488) (end 130.81 103.378) (width 0.254) (layer F.Cu) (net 15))
 (via (at 130.81 103.378) (size 0.762) (drill 0.381) (layers F.Cu B.Cu) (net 15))
 (segment (start 123.698 103.378) (end 120.65 100.33) (width 0.254) (layer B.Cu) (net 15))
 (segment (start 130.81 103.378) (end 123.698 103.378) (width 0.254) (layer B.Cu) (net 15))
 (segment (start 140.081001 94.106999) (end 139.7 94.488) (width 0.254) (layer F.Cu) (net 15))
 (segment (start 140.081001 91.312999) (end 140.081001 94.106999) (width 0.254) (layer F.Cu) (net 15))
 (segment (start 140.462 90.932) (end 140.081001 91.312999) (width 0.254) (layer F.Cu) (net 15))
 (segment (start 127.254 103.886) (end 135.128 111.76) (width 0.254) (layer F.Cu) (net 16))
 (segment (start 127.254 93.726) (end 127.254 103.886) (width 0.254) (layer F.Cu) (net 16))
 (segment (start 130.81 92.71) (end 128.27 92.71) (width 0.254) (layer F.Cu) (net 16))
 (segment (start 128.27 92.71) (end 127.254 93.726) (width 0.254) (layer F.Cu) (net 16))
 (segment (start 156.027999 100.655999) (end 157.154001 100.655999) (width 0.254) (layer B.Cu) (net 16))
 (segment (start 155.448 100.076) (end 156.027999 100.655999) (width 0.254) (layer B.Cu) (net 16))
 (segment (start 157.154001 100.655999) (end 157.734 100.076) (width 0.254) (layer B.Cu) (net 16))
 (segment (start 157.734 95.859718) (end 154.584282 92.71) (width 0.254) (layer B.Cu) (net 16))
 (segment (start 157.734 100.076) (end 157.734 95.859718) (width 0.254) (layer B.Cu) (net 16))
 (segment (start 154.584282 92.71) (end 142.24 92.71) (width 0.254) (layer B.Cu) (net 16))
 (segment (start 142.24 92.71) (end 130.81 92.71) (width 0.254) (layer B.Cu) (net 16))
 (segment (start 143.764 81.026) (end 132.08 69.342) (width 0.254) (layer F.Cu) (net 21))
 (segment (start 147.668 81.026) (end 143.764 81.026) (width 0.254) (layer F.Cu) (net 21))
 (segment (start 143.764 83.566) (end 129.54 69.342) (width 0.254) (layer B.Cu) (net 22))
 (segment (start 147.668 83.566) (end 143.764 83.566) (width 0.254) (layer B.Cu) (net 22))
 (segment (start 154.661999 87.052001) (end 133.280001 87.052001) (width 0.254) (layer F.Cu) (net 23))
 (segment (start 155.608 86.106) (end 154.661999 87.052001) (width 0.254) (layer F.Cu) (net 23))
 (segment (start 132.08 85.852) (end 132.08 84.582) (width 0.254) (layer F.Cu) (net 23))
 (segment (start 133.280001 87.052001) (end 132.08 85.852) (width 0.254) (layer F.Cu) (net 23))
 (segment (start 155.043001 81.590999) (end 148.787001 81.590999) (width 0.254) (layer F.Cu) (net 25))
 (segment (start 155.608 81.026) (end 155.043001 81.590999) (width 0.254) (layer F.Cu) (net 25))
 (segment (start 130.428999 83.693001) (end 129.54 84.582) (width 0.254) (layer F.Cu) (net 25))
 (segment (start 132.149999 81.972001) (end 130.428999 83.693001) (width 0.254) (layer F.Cu) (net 25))
 (segment (start 148.405999 81.972001) (end 132.149999 81.972001) (width 0.254) (layer F.Cu) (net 25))
 (segment (start 148.787001 81.590999) (end 148.405999 81.972001) (width 0.254) (layer F.Cu) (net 25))
 (segment (start 140.588999 70.230999) (end 139.7 69.342) (width 0.254) (layer F.Cu) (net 26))
 (segment (start 144.710001 74.352001) (end 140.588999 70.230999) (width 0.254) (layer F.Cu) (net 26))
 (segment (start 151.474001 74.352001) (end 144.710001 74.352001) (width 0.254) (layer F.Cu) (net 26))
 (segment (start 155.608 78.486) (end 151.474001 74.352001) (width 0.254) (layer F.Cu) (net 26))
 (segment (start 137.16 83.324765) (end 138.004754 82.480011) (width 0.254) (layer F.Cu) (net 27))
 (segment (start 137.16 84.582) (end 137.16 83.324765) (width 0.254) (layer F.Cu) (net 27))
 (segment (start 138.004754 82.480011) (end 156.279989 82.480011) (width 0.254) (layer F.Cu) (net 27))
 (segment (start 156.279989 82.480011) (end 156.972 82.042) (width 0.254) (layer F.Cu) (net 27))
 (segment (start 156.972 82.042) (end 156.972 76.962) (width 0.254) (layer F.Cu) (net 27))
 (segment (start 156.520999 76.510999) (end 156.972 76.962) (width 0.254) (layer F.Cu) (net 27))
 (segment (start 156.172999 76.510999) (end 156.520999 76.510999) (width 0.254) (layer F.Cu) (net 27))
 (segment (start 155.608 75.946) (end 156.172999 76.510999) (width 0.254) (layer F.Cu) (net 27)))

